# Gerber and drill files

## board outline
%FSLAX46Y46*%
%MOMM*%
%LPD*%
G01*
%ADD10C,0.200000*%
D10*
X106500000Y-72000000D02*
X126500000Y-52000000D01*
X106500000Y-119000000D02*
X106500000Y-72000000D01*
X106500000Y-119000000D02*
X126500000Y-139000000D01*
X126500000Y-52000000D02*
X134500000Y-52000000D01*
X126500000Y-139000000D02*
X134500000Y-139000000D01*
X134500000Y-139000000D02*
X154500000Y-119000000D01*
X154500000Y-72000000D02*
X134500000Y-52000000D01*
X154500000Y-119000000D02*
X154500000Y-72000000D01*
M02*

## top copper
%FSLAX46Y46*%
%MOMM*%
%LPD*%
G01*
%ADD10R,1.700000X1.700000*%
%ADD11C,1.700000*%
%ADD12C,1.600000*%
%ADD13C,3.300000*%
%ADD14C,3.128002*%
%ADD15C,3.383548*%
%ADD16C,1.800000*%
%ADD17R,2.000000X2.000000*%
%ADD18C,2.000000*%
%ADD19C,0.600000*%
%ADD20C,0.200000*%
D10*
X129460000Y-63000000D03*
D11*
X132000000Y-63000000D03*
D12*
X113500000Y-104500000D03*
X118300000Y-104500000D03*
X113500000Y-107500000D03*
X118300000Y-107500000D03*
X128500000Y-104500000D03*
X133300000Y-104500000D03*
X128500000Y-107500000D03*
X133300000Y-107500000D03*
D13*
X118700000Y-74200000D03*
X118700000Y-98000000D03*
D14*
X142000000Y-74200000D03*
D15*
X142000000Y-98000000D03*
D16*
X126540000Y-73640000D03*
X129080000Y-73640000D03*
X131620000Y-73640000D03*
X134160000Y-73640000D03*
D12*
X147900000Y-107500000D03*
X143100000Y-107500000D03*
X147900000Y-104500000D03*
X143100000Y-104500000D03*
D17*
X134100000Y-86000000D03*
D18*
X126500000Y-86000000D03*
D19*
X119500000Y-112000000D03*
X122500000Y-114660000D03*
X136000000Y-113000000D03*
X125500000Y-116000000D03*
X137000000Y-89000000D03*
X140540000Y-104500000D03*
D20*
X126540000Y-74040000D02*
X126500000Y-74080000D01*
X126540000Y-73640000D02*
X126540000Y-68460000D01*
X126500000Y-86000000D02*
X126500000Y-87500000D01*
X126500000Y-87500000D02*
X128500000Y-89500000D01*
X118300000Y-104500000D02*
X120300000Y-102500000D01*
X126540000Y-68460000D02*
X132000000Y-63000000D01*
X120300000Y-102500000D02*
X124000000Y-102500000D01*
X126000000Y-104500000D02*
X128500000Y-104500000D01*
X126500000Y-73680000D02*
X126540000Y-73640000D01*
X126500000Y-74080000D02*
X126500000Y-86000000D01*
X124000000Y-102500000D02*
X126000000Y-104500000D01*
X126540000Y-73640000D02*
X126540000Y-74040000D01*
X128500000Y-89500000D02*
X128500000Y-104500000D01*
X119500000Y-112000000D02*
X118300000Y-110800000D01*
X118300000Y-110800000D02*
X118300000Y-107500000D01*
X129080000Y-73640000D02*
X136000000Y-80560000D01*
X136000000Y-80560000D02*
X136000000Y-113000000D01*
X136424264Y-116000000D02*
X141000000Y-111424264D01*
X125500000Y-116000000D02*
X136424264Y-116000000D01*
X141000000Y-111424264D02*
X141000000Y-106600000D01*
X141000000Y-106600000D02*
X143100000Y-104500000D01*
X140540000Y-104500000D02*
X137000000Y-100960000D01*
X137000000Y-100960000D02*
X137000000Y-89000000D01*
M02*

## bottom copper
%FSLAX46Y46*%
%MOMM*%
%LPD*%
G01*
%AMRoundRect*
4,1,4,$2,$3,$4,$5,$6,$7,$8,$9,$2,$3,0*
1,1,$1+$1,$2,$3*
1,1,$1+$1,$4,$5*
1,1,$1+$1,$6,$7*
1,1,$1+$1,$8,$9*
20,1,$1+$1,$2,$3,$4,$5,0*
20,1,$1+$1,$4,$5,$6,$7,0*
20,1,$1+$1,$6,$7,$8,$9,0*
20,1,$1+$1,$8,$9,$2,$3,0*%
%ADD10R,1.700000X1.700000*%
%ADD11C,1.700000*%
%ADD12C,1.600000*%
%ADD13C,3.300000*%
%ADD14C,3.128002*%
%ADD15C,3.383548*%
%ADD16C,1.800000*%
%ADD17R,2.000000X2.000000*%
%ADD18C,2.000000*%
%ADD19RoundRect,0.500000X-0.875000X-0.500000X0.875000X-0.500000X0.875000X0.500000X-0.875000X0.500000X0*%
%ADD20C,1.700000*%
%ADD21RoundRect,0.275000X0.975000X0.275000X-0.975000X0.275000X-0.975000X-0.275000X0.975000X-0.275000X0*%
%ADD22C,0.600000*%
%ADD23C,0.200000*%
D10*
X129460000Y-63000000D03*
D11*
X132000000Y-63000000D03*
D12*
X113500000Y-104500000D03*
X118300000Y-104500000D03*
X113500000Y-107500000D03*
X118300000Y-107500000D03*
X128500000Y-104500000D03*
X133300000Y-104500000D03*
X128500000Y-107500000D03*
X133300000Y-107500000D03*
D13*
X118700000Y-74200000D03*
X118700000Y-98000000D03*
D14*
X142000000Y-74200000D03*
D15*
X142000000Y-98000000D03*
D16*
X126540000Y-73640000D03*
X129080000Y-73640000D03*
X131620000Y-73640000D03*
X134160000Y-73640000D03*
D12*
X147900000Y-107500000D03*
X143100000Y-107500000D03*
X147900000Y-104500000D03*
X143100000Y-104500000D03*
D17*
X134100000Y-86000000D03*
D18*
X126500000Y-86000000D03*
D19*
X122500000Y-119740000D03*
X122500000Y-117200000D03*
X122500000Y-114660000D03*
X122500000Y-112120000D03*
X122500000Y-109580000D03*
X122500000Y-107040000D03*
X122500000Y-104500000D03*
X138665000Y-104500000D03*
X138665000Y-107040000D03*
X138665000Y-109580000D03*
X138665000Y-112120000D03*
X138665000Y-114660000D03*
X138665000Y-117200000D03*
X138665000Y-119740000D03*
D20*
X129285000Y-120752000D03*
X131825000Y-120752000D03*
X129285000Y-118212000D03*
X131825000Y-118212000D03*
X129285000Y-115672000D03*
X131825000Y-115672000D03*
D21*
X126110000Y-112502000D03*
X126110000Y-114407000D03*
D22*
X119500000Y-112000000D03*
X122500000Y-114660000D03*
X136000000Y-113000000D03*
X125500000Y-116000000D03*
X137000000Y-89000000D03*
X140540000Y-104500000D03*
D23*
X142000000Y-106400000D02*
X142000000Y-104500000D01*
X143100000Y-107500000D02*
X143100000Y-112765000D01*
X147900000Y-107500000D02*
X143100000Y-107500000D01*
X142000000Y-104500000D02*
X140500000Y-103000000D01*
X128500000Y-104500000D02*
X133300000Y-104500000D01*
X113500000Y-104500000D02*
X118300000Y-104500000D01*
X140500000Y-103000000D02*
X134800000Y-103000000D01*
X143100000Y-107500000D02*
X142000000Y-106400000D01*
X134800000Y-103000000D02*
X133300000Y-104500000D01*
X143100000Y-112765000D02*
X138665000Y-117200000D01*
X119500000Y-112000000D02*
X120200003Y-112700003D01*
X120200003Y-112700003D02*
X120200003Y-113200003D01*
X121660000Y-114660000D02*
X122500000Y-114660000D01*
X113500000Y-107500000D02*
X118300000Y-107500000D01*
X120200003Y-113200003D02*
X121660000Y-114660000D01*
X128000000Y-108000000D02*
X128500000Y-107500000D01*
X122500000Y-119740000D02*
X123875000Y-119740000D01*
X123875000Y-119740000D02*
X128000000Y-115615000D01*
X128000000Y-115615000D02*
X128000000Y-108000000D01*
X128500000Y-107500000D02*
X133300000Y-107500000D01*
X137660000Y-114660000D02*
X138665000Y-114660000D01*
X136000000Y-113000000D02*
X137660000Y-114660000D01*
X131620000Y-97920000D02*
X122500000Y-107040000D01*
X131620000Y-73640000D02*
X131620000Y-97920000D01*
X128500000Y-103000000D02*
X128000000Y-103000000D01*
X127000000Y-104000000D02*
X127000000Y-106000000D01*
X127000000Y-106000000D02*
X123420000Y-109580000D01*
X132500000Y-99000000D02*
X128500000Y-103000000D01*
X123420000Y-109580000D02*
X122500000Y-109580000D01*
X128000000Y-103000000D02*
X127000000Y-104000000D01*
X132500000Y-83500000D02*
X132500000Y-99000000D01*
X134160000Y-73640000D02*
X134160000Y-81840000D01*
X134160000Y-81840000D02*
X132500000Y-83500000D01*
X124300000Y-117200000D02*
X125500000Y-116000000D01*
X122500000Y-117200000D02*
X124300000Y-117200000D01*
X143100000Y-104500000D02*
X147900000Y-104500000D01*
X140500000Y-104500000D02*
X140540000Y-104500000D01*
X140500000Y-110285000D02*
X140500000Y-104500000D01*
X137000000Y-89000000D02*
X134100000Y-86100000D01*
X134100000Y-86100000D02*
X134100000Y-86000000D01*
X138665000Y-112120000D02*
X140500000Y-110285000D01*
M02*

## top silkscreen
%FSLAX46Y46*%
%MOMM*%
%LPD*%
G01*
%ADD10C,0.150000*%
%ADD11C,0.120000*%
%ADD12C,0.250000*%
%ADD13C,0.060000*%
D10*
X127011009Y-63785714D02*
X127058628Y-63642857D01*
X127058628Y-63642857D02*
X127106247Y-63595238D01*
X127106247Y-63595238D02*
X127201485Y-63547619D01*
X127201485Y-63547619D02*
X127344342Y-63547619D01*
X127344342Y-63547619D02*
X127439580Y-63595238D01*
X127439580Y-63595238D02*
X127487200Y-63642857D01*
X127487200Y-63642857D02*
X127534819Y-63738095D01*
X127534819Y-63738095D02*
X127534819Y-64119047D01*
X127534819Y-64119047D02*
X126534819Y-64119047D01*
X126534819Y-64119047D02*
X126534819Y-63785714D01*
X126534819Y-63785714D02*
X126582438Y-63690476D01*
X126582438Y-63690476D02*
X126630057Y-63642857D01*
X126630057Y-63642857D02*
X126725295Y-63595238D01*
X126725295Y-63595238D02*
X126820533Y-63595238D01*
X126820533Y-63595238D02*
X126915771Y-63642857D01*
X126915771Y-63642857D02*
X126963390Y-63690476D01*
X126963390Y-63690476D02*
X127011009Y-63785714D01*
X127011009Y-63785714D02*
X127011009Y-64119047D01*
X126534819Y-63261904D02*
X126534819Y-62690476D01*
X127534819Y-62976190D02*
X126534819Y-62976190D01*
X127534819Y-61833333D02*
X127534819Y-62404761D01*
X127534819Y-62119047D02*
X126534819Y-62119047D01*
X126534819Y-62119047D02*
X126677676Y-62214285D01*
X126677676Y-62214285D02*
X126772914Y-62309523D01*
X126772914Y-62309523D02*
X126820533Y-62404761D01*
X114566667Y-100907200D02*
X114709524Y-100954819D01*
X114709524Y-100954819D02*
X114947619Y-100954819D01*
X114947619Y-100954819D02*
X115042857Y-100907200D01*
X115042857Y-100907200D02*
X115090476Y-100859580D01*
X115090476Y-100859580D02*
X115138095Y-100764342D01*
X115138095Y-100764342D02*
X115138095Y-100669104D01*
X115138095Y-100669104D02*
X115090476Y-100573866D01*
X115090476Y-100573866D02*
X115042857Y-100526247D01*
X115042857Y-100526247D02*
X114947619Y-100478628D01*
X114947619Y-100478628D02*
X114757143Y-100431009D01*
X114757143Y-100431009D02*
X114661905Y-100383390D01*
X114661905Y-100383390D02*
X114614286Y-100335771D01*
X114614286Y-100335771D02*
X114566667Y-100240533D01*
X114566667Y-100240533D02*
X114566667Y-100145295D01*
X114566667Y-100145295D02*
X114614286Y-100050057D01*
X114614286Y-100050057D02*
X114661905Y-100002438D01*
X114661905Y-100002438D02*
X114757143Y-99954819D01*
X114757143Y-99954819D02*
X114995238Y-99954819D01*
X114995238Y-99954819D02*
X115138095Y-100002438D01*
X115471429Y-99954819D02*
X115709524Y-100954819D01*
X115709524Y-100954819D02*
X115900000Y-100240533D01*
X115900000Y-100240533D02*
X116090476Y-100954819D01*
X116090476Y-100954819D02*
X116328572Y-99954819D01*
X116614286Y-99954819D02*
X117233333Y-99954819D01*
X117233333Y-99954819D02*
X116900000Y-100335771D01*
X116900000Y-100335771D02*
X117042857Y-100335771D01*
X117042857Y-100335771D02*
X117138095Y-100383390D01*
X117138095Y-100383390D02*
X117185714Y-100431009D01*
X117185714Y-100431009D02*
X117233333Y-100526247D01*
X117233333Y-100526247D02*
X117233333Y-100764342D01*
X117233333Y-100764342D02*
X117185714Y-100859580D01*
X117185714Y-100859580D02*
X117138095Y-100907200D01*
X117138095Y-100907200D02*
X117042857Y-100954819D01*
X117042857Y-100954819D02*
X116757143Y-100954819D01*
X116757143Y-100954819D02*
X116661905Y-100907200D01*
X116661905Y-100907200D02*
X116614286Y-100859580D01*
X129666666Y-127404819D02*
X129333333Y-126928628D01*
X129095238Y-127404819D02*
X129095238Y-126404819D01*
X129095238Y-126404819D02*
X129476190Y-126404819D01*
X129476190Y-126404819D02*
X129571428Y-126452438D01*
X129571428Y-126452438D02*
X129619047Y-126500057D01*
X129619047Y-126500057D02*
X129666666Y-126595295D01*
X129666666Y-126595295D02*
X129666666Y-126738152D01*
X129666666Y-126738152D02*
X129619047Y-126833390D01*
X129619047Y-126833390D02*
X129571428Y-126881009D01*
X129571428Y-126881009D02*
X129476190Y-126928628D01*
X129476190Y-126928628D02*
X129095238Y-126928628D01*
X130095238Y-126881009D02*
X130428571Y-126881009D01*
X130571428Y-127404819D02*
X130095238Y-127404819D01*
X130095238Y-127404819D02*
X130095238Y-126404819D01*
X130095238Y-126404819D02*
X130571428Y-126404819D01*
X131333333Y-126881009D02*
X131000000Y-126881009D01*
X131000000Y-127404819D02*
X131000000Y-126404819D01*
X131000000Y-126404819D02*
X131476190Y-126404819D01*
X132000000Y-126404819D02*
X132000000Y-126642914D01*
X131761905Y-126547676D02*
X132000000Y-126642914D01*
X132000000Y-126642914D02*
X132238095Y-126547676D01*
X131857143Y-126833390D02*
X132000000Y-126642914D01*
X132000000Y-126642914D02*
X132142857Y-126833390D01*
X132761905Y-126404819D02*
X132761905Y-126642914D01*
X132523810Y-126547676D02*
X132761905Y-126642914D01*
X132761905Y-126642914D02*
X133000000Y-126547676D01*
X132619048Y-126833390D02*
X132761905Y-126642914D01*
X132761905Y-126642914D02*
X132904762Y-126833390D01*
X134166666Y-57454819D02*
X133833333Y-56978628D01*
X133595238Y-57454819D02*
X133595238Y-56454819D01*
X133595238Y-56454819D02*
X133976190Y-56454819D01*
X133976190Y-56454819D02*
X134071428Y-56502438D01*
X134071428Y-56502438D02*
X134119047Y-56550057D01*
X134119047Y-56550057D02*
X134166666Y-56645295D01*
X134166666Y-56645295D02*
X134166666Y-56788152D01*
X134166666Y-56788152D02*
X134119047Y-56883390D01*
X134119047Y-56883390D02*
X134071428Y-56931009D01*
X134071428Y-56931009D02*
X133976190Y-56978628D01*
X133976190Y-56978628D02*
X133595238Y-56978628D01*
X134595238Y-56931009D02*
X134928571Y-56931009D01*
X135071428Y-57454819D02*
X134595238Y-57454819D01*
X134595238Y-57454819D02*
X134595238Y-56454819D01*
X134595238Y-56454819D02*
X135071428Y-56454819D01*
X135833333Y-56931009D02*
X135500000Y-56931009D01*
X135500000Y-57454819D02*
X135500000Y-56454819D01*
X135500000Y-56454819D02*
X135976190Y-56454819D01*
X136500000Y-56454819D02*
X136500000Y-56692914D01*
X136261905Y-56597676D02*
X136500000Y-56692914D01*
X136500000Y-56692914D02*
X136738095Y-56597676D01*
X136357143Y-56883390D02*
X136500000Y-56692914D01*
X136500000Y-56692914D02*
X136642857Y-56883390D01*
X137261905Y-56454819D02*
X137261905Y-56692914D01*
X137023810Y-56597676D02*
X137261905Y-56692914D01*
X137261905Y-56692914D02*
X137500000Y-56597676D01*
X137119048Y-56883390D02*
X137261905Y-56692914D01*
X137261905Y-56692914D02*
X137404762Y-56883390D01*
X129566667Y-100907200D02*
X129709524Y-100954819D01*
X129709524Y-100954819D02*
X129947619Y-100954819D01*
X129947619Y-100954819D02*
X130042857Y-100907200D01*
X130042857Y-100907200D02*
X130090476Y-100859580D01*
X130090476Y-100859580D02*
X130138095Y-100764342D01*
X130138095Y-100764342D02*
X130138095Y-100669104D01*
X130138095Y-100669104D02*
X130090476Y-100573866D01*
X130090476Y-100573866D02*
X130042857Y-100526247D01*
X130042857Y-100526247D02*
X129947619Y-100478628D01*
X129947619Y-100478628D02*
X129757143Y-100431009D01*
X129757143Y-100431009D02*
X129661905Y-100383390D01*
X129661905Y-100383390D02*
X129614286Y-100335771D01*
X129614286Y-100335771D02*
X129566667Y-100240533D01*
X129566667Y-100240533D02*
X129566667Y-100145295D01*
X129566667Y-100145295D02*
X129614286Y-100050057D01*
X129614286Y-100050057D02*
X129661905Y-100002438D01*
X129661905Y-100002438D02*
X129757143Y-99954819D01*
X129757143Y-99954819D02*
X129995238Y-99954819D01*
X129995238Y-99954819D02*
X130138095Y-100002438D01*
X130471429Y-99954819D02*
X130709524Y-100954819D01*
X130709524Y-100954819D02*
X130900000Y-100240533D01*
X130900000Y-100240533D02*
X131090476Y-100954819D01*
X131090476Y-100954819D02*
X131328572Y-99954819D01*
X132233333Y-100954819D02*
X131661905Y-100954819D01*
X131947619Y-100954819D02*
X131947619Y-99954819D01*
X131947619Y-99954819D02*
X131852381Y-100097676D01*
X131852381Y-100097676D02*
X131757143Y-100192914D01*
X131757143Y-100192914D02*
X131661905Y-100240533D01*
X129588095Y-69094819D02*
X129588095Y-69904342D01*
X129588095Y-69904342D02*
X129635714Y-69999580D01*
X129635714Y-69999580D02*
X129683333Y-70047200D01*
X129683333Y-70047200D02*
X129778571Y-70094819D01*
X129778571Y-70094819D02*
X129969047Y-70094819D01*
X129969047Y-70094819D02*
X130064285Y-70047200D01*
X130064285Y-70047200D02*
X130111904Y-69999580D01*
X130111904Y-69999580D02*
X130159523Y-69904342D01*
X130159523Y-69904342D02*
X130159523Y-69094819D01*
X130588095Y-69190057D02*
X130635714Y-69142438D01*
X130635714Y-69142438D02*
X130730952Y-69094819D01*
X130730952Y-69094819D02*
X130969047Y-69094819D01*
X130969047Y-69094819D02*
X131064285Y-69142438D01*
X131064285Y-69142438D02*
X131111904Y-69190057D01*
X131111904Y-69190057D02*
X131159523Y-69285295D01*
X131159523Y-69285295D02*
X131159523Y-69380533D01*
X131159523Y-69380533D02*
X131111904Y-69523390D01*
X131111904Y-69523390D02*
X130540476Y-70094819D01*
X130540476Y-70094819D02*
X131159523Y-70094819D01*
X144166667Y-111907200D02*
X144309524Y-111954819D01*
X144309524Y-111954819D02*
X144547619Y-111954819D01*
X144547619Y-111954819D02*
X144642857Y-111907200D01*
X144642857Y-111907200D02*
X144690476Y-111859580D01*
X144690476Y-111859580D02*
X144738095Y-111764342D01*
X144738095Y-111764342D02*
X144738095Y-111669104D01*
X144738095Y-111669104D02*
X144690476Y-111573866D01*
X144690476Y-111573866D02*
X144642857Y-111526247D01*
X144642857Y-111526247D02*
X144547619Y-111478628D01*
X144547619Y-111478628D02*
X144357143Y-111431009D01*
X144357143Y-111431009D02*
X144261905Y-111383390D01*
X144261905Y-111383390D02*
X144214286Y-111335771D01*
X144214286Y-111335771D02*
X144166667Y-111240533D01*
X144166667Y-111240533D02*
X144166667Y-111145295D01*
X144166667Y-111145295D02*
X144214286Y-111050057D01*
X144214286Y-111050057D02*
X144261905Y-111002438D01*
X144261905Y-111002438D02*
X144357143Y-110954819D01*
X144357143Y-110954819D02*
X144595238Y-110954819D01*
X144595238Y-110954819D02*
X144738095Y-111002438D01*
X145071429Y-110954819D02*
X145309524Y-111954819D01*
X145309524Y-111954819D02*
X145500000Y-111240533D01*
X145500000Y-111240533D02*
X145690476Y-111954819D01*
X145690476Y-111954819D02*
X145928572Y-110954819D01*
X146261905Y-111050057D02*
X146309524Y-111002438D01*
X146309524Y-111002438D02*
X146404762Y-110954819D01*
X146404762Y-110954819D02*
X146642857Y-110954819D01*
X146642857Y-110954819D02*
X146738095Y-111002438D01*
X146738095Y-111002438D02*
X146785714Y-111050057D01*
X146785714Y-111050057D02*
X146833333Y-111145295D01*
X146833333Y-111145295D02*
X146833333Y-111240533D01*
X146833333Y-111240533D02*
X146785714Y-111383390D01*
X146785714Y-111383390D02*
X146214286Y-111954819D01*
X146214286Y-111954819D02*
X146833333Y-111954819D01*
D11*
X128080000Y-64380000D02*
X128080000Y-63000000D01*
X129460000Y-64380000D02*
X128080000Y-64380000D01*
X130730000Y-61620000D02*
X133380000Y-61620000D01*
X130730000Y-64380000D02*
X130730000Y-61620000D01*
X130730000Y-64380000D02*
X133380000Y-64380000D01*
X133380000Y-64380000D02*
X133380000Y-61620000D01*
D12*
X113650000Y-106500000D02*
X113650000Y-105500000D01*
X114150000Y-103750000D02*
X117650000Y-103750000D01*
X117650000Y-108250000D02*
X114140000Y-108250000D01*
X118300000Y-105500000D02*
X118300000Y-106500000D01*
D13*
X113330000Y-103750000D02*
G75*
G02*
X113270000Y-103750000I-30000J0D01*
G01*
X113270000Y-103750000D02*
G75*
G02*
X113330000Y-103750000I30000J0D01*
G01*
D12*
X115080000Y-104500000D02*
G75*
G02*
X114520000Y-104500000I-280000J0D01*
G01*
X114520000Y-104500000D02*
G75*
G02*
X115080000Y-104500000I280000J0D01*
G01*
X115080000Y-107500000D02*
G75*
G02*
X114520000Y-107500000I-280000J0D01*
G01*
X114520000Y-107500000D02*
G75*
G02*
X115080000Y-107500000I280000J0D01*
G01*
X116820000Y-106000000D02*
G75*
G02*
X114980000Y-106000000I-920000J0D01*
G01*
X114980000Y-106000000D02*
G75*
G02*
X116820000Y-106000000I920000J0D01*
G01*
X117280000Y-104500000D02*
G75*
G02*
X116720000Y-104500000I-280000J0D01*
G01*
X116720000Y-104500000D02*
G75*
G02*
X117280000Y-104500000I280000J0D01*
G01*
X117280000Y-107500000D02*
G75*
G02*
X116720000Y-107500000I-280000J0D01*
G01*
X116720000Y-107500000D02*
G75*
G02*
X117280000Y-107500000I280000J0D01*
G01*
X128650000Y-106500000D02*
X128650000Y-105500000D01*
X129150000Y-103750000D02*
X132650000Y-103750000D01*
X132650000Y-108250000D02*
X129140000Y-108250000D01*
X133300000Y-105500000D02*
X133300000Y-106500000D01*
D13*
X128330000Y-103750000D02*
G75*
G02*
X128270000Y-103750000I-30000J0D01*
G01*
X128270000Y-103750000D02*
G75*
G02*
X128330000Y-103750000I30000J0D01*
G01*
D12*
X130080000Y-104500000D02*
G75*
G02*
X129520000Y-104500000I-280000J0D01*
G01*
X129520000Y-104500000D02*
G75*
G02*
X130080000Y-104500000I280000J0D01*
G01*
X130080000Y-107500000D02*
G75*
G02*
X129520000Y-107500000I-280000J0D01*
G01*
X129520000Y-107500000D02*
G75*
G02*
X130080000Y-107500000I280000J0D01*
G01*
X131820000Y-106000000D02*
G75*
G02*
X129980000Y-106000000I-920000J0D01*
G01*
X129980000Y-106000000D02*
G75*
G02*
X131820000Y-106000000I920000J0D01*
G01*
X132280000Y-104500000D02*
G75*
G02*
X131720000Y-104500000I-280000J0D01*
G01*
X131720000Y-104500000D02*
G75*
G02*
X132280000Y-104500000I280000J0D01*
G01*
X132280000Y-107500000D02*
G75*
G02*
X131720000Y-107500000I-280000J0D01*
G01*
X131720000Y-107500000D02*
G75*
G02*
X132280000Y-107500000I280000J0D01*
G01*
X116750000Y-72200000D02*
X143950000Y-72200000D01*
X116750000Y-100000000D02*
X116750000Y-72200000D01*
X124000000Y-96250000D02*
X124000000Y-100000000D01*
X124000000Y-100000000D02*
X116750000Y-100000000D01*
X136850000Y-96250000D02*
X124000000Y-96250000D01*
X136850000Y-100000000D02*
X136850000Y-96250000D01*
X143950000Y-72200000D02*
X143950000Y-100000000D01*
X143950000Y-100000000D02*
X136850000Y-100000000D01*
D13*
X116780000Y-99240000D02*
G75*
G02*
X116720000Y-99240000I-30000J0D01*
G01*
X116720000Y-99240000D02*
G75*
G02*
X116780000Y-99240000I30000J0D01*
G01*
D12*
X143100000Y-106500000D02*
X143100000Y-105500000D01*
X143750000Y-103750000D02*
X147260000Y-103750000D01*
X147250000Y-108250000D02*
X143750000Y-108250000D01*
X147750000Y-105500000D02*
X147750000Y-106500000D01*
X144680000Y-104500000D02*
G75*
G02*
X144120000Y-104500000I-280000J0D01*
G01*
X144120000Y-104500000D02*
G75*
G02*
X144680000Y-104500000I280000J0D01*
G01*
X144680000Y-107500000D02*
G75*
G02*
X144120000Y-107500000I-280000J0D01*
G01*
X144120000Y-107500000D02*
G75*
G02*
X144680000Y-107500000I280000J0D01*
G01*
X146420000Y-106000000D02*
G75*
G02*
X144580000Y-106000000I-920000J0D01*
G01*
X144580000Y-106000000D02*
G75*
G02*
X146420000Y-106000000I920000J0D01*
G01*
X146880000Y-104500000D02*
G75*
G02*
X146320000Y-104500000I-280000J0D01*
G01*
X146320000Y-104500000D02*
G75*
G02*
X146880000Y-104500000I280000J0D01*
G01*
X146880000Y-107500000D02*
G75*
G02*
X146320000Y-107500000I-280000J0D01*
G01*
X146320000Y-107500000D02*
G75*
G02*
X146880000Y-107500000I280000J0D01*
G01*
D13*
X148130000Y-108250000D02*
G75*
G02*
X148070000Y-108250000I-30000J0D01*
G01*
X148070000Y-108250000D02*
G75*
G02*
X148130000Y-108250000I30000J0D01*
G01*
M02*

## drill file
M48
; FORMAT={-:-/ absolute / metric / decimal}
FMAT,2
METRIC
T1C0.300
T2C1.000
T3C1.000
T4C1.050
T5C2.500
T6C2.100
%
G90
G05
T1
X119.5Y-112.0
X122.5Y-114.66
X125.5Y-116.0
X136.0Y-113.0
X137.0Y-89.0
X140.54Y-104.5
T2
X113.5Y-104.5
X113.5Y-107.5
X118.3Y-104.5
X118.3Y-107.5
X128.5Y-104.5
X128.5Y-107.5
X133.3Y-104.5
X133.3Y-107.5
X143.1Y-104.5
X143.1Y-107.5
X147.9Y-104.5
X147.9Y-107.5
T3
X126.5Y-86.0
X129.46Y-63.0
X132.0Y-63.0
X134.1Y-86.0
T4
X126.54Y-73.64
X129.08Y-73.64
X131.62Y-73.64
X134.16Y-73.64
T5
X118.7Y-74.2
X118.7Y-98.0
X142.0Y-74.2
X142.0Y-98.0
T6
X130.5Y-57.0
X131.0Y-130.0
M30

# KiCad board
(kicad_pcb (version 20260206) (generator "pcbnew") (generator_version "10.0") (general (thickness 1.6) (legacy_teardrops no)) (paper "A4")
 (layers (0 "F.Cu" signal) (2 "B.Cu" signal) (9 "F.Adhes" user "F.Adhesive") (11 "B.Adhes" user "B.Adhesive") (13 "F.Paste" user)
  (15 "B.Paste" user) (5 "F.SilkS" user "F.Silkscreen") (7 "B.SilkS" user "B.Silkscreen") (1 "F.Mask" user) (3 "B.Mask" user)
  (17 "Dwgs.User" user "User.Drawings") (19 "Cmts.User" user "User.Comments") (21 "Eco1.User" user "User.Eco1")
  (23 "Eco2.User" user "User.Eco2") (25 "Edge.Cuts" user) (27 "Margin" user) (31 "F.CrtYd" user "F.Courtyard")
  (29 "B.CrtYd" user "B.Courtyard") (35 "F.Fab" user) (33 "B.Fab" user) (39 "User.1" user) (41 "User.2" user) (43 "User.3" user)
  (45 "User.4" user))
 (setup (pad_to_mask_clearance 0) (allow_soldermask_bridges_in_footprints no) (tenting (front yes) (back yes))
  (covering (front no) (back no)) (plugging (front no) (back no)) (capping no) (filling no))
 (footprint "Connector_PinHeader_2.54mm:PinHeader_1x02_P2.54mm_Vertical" (layer "F.Cu") (at 129.46 63 90)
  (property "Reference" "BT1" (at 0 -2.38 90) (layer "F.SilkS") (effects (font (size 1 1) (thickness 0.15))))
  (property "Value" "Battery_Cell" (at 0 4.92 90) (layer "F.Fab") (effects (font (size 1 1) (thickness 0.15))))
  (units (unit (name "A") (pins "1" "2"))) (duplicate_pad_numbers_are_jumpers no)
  (fp_line (start -1.38 -1.38) (end 0 -1.38) (stroke (width 0.12) (type solid)) (layer "F.SilkS"))
  (fp_line (start -1.38 0) (end -1.38 -1.38) (stroke (width 0.12) (type solid)) (layer "F.SilkS"))
  (fp_line (start 1.38 1.27) (end 1.38 3.92) (stroke (width 0.12) (type solid)) (layer "F.SilkS"))
  (fp_line (start -1.38 1.27) (end 1.38 1.27) (stroke (width 0.12) (type solid)) (layer "F.SilkS"))
  (fp_line (start -1.38 1.27) (end -1.38 3.92) (stroke (width 0.12) (type solid)) (layer "F.SilkS"))
  (fp_line (start -1.38 3.92) (end 1.38 3.92) (stroke (width 0.12) (type solid)) (layer "F.SilkS"))
  (pad "1" thru_hole rect (at 0 0 90) (size 1.7 1.7) (drill 1) (layers "*.Cu" "*.Mask") (remove_unused_layers no) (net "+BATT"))
  (pad "2" thru_hole circle (at 0 2.54 90) (size 1.7 1.7) (drill 1) (layers "*.Cu" "*.Mask") (remove_unused_layers no) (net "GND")))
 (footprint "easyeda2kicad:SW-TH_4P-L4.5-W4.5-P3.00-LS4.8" (layer "F.Cu") (at 115.9 106)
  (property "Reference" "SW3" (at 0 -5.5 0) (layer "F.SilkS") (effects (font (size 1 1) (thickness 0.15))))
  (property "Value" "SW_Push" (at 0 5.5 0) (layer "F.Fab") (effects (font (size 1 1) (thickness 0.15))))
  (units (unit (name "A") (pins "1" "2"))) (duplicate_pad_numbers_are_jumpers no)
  (fp_line (start -2.25 0.5) (end -2.25 -0.5) (stroke (width 0.25) (type solid)) (layer "F.SilkS"))
  (fp_line (start -1.75 -2.25) (end 1.75 -2.25) (stroke (width 0.25) (type solid)) (layer "F.SilkS"))
  (fp_line (start 1.75 2.25) (end -1.76 2.25) (stroke (width 0.25) (type solid)) (layer "F.SilkS"))
  (fp_line (start 2.4 -0.5) (end 2.4 0.5) (stroke (width 0.25) (type solid)) (layer "F.SilkS"))
  (fp_circle (center -2.6 -2.25) (end -2.57 -2.25) (stroke (width 0.06) (type solid)) (fill no) (layer "F.SilkS"))
  (fp_circle (center -1.1 -1.5) (end -0.82 -1.5) (stroke (width 0.25) (type solid)) (fill no) (layer "F.SilkS"))
  (fp_circle (center -1.1 1.5) (end -0.82 1.5) (stroke (width 0.25) (type solid)) (fill no) (layer "F.SilkS"))
  (fp_circle (center 0 0) (end 0.92 0) (stroke (width 0.25) (type solid)) (fill no) (layer "F.SilkS"))
  (fp_circle (center 1.1 -1.5) (end 1.38 -1.5) (stroke (width 0.25) (type solid)) (fill no) (layer "F.SilkS"))
  (fp_circle (center 1.1 1.5) (end 1.38 1.5) (stroke (width 0.25) (type solid)) (fill no) (layer "F.SilkS"))
  (pad "1" thru_hole circle (at -2.4 -1.5) (size 1.6 1.6) (drill 0.999998) (layers "*.Cu" "*.Mask") (remove_unused_layers no) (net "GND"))
  (pad "1" thru_hole circle (at 2.4 -1.5) (size 1.6 1.6) (drill 0.999998) (layers "*.Cu" "*.Mask") (remove_unused_layers no) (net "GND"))
  (pad "2" thru_hole circle (at -2.4 1.5) (size 1.6 1.6) (drill 0.999998) (layers "*.Cu" "*.Mask") (remove_unused_layers no)
   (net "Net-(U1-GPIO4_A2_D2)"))
  (pad "2" thru_hole circle (at 2.4 1.5) (size 1.6 1.6) (drill 0.999998) (layers "*.Cu" "*.Mask") (remove_unused_layers no)
   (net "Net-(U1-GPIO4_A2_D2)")))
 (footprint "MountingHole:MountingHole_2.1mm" (layer "F.Cu") (at 131 130)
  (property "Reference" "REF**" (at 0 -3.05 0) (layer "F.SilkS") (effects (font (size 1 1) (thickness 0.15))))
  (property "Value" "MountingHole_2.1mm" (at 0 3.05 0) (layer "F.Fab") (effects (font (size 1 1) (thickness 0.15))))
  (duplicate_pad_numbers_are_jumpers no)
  (pad "" np_thru_hole circle (at 0 0) (size 2.1 2.1) (drill 2.1) (layers "*.Cu" "*.Mask")))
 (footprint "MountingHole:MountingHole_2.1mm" (layer "F.Cu") (at 130.5 57)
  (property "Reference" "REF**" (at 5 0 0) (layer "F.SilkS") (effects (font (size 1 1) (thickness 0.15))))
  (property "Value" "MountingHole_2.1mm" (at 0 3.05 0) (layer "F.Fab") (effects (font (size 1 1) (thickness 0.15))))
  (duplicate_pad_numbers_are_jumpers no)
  (pad "" np_thru_hole circle (at 0 0) (size 2.1 2.1) (drill 2.1) (layers "*.Cu" "*.Mask")))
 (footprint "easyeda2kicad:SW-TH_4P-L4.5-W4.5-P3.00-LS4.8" (layer "F.Cu") (at 130.9 106)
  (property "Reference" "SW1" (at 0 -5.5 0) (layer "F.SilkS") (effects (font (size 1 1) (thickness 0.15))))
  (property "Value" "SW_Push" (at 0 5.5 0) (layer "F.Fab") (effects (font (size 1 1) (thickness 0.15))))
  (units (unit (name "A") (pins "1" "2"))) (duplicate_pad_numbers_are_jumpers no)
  (fp_line (start -2.25 0.5) (end -2.25 -0.5) (stroke (width 0.25) (type solid)) (layer "F.SilkS"))
  (fp_line (start -1.75 -2.25) (end 1.75 -2.25) (stroke (width 0.25) (type solid)) (layer "F.SilkS"))
  (fp_line (start 1.75 2.25) (end -1.76 2.25) (stroke (width 0.25) (type solid)) (layer "F.SilkS"))
  (fp_line (start 2.4 -0.5) (end 2.4 0.5) (stroke (width 0.25) (type solid)) (layer "F.SilkS"))
  (fp_circle (center -2.6 -2.25) (end -2.57 -2.25) (stroke (width 0.06) (type solid)) (fill no) (layer "F.SilkS"))
  (fp_circle (center -1.1 -1.5) (end -0.82 -1.5) (stroke (width 0.25) (type solid)) (fill no) (layer "F.SilkS"))
  (fp_circle (center -1.1 1.5) (end -0.82 1.5) (stroke (width 0.25) (type solid)) (fill no) (layer "F.SilkS"))
  (fp_circle (center 0 0) (end 0.92 0) (stroke (width 0.25) (type solid)) (fill no) (layer "F.SilkS"))
  (fp_circle (center 1.1 -1.5) (end 1.38 -1.5) (stroke (width 0.25) (type solid)) (fill no) (layer "F.SilkS"))
  (fp_circle (center 1.1 1.5) (end 1.38 1.5) (stroke (width 0.25) (type solid)) (fill no) (layer "F.SilkS"))
  (pad "1" thru_hole circle (at -2.4 -1.5) (size 1.6 1.6) (drill 0.999998) (layers "*.Cu" "*.Mask") (remove_unused_layers no) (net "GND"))
  (pad "1" thru_hole circle (at 2.4 -1.5) (size 1.6 1.6) (drill 0.999998) (layers "*.Cu" "*.Mask") (remove_unused_layers no) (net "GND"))
  (pad "2" thru_hole circle (at -2.4 1.5) (size 1.6 1.6) (drill 0.999998) (layers "*.Cu" "*.Mask") (remove_unused_layers no)
   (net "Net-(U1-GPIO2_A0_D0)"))
  (pad "2" thru_hole circle (at 2.4 1.5) (size 1.6 1.6) (drill 0.999998) (layers "*.Cu" "*.Mask") (remove_unused_layers no)
   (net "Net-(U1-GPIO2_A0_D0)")))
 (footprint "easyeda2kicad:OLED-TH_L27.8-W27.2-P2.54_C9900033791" (layer "F.Cu") (at 130.35 73.64)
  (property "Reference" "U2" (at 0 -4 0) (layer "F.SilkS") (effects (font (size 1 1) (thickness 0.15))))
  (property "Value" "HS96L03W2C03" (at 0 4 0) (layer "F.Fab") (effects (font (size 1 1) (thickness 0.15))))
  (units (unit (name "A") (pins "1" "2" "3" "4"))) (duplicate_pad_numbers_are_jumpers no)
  (fp_line (start -13.6 -1.44) (end 13.6 -1.44) (stroke (width 0.25) (type solid)) (layer "F.SilkS"))
  (fp_line (start -13.6 26.36) (end -13.6 -1.44) (stroke (width 0.25) (type solid)) (layer "F.SilkS"))
  (fp_line (start -6.35 22.61) (end -6.35 26.36) (stroke (width 0.25) (type solid)) (layer "F.SilkS"))
  (fp_line (start -6.35 26.36) (end -13.6 26.36) (stroke (width 0.25) (type solid)) (layer "F.SilkS"))
  (fp_line (start 6.5 22.61) (end -6.35 22.61) (stroke (width 0.25) (type solid)) (layer "F.SilkS"))
  (fp_line (start 6.5 26.36) (end 6.5 22.61) (stroke (width 0.25) (type solid)) (layer "F.SilkS"))
  (fp_line (start 13.6 -1.44) (end 13.6 26.36) (stroke (width 0.25) (type solid)) (layer "F.SilkS"))
  (fp_line (start 13.6 26.36) (end 6.5 26.36) (stroke (width 0.25) (type solid)) (layer "F.SilkS"))
  (fp_circle (center -13.6 25.6) (end -13.57 25.6) (stroke (width 0.06) (type solid)) (fill no) (layer "F.SilkS"))
  (pad "" thru_hole circle (at -11.65 0.56) (size 3.3 3.3) (drill 2.5) (layers "*.Cu" "*.Mask") (remove_unused_layers no))
  (pad "" thru_hole circle (at -11.65 24.36) (size 3.3 3.3) (drill 2.5) (layers "*.Cu" "*.Mask") (remove_unused_layers no))
  (pad "" thru_hole circle (at 11.65 0.56) (size 3.128002 3.128002) (drill 2.5) (layers "*.Cu" "*.Mask") (remove_unused_layers no))
  (pad "" thru_hole circle (at 11.65 24.36) (size 3.383548 3.383548) (drill 2.5) (layers "*.Cu" "*.Mask") (remove_unused_layers no))
  (pad "1" thru_hole circle (at -3.81 0) (size 1.8 1.8) (drill 1.049986) (layers "*.Cu" "*.Mask") (remove_unused_layers no) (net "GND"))
  (pad "2" thru_hole circle (at -1.27 0) (size 1.8 1.8) (drill 1.049986) (layers "*.Cu" "*.Mask") (remove_unused_layers no) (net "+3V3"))
  (pad "3" thru_hole circle (at 1.27 0) (size 1.8 1.8) (drill 1.049986) (layers "*.Cu" "*.Mask") (remove_unused_layers no)
   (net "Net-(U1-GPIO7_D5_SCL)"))
  (pad "4" thru_hole circle (at 3.81 0) (size 1.8 1.8) (drill 1.049986) (layers "*.Cu" "*.Mask") (remove_unused_layers no)
   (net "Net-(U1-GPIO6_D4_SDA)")))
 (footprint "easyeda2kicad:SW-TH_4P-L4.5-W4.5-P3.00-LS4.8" (layer "F.Cu") (at 145.5 106 180)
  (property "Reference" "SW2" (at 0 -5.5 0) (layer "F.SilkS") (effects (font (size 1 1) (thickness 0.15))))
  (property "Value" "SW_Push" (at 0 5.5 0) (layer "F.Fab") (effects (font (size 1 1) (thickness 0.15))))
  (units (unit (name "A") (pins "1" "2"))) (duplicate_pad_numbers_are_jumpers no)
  (fp_line (start 2.4 -0.5) (end 2.4 0.5) (stroke (width 0.25) (type solid)) (layer "F.SilkS"))
  (fp_line (start 1.75 2.25) (end -1.76 2.25) (stroke (width 0.25) (type solid)) (layer "F.SilkS"))
  (fp_line (start -1.75 -2.25) (end 1.75 -2.25) (stroke (width 0.25) (type solid)) (layer "F.SilkS"))
  (fp_line (start -2.25 0.5) (end -2.25 -0.5) (stroke (width 0.25) (type solid)) (layer "F.SilkS"))
  (fp_circle (center 1.1 1.5) (end 1.38 1.5) (stroke (width 0.25) (type solid)) (fill no) (layer "F.SilkS"))
  (fp_circle (center 1.1 -1.5) (end 1.38 -1.5) (stroke (width 0.25) (type solid)) (fill no) (layer "F.SilkS"))
  (fp_circle (center 0 0) (end 0.92 0) (stroke (width 0.25) (type solid)) (fill no) (layer "F.SilkS"))
  (fp_circle (center -1.1 1.5) (end -0.82 1.5) (stroke (width 0.25) (type solid)) (fill no) (layer "F.SilkS"))
  (fp_circle (center -1.1 -1.5) (end -0.82 -1.5) (stroke (width 0.25) (type solid)) (fill no) (layer "F.SilkS"))
  (fp_circle (center -2.6 -2.25) (end -2.57 -2.25) (stroke (width 0.06) (type solid)) (fill no) (layer "F.SilkS"))
  (pad "1" thru_hole circle (at -2.4 -1.5 180) (size 1.6 1.6) (drill 0.999998) (layers "*.Cu" "*.Mask") (remove_unused_layers no)
   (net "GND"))
  (pad "1" thru_hole circle (at 2.4 -1.5 180) (size 1.6 1.6) (drill 0.999998) (layers "*.Cu" "*.Mask") (remove_unused_layers no) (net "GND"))
  (pad "2" thru_hole circle (at -2.4 1.5 180) (size 1.6 1.6) (drill 0.999998) (layers "*.Cu" "*.Mask") (remove_unused_layers no)
   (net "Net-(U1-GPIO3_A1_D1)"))
  (pad "2" thru_hole circle (at 2.4 1.5 180) (size 1.6 1.6) (drill 0.999998) (layers "*.Cu" "*.Mask") (remove_unused_layers no)
   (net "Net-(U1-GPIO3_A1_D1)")))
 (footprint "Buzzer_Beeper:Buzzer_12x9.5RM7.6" (layer "B.Cu") (at 134.1 86 180)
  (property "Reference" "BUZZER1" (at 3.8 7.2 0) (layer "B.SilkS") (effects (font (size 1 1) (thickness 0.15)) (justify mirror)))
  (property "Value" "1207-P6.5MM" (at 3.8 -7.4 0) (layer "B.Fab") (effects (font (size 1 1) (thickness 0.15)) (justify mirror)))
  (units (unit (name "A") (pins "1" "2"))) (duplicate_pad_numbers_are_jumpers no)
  (pad "1" thru_hole rect (at 0 0 180) (size 2 2) (drill 1) (layers "*.Cu" "*.Mask") (remove_unused_layers no) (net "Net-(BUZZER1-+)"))
  (pad "2" thru_hole circle (at 7.6 0 180) (size 2 2) (drill 1) (layers "*.Cu" "*.Mask") (remove_unused_layers no) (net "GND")))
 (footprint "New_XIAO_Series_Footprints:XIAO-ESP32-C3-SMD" (layer "B.Cu") (at 121.665 101.62)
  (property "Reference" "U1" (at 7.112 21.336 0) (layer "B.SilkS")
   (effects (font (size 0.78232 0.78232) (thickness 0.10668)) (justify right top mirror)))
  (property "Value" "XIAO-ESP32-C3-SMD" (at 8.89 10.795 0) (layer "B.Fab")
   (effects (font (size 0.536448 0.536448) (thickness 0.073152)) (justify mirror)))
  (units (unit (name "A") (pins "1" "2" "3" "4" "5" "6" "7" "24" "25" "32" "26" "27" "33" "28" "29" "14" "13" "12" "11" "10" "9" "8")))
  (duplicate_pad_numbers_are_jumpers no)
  (pad "1" smd roundrect (at 0.835 18.12) (size 2.75 2) (layers "B.Cu" "B.Mask" "B.Paste") (roundrect_rratio 0.25)
   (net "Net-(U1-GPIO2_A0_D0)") (solder_mask_margin 0.0508) (thermal_bridge_angle 45))
  (pad "2" smd roundrect (at 0.835 15.58) (size 2.75 2) (layers "B.Cu" "B.Mask" "B.Paste") (roundrect_rratio 0.25)
   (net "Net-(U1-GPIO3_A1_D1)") (solder_mask_margin 0.0508) (thermal_bridge_angle 45))
  (pad "3" smd roundrect (at 0.835 13.04) (size 2.75 2) (layers "B.Cu" "B.Mask" "B.Paste") (roundrect_rratio 0.25)
   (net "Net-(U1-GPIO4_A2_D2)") (solder_mask_margin 0.0508) (thermal_bridge_angle 45))
  (pad "4" smd roundrect (at 0.835 10.5) (size 2.75 2) (layers "B.Cu" "B.Mask" "B.Paste") (roundrect_rratio 0.25)
   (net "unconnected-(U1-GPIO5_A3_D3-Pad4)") (solder_mask_margin 0.0508) (thermal_bridge_angle 45))
  (pad "5" smd roundrect (at 0.835 7.96) (size 2.75 2) (layers "B.Cu" "B.Mask" "B.Paste") (roundrect_rratio 0.25)
   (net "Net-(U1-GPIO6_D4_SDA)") (solder_mask_margin 0.0508) (thermal_bridge_angle 45))
  (pad "6" smd roundrect (at 0.835 5.42) (size 2.75 2) (layers "B.Cu" "B.Mask" "B.Paste") (roundrect_rratio 0.25)
   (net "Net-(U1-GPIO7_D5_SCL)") (solder_mask_margin 0.0508) (thermal_bridge_angle 45))
  (pad "7" smd roundrect (at 0.835 2.88) (size 2.75 2) (layers "B.Cu" "B.Mask" "B.Paste") (roundrect_rratio 0.25)
   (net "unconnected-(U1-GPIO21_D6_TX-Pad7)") (solder_mask_margin 0.0508) (thermal_bridge_angle 45))
  (pad "8" smd roundrect (at 17 2.88) (size 2.75 2) (layers "B.Cu" "B.Mask" "B.Paste") (roundrect_rratio 0.25)
   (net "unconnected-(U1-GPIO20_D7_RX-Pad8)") (solder_mask_margin 0.0508) (thermal_bridge_angle 45))
  (pad "9" smd roundrect (at 17 5.42) (size 2.75 2) (layers "B.Cu" "B.Mask" "B.Paste") (roundrect_rratio 0.25)
   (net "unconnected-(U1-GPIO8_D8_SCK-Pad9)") (solder_mask_margin 0.0508) (thermal_bridge_angle 45))
  (pad "10" smd roundrect (at 17 7.96) (size 2.75 2) (layers "B.Cu" "B.Mask" "B.Paste") (roundrect_rratio 0.25)
   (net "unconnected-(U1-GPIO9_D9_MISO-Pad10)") (solder_mask_margin 0.0508) (thermal_bridge_angle 45))
  (pad "11" smd roundrect (at 17 10.5) (size 2.75 2) (layers "B.Cu" "B.Mask" "B.Paste") (roundrect_rratio 0.25) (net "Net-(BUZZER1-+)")
   (solder_mask_margin 0.0508) (thermal_bridge_angle 45))
  (pad "12" smd roundrect (at 17 13.04) (size 2.75 2) (layers "B.Cu" "B.Mask" "B.Paste") (roundrect_rratio 0.25) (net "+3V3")
   (solder_mask_margin 0.0508) (thermal_bridge_angle 45))
  (pad "13" smd roundrect (at 17 15.58) (size 2.75 2) (layers "B.Cu" "B.Mask" "B.Paste") (roundrect_rratio 0.25) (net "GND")
   (solder_mask_margin 0.0508) (thermal_bridge_angle 45))
  (pad "14" smd roundrect (at 17 18.12) (size 2.75 2) (layers "B.Cu" "B.Mask" "B.Paste") (roundrect_rratio 0.25) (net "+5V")
   (solder_mask_margin 0.0508) (thermal_bridge_angle 45))
  (pad "15" smd circle (at 7.62 19.132) (size 1.7 1.7) (layers "B.Cu" "B.Mask" "B.Paste"))
  (pad "16" smd circle (at 10.16 19.132) (size 1.7 1.7) (layers "B.Cu" "B.Mask" "B.Paste"))
  (pad "17" smd circle (at 7.62 16.592) (size 1.7 1.7) (layers "B.Cu" "B.Mask" "B.Paste"))
  (pad "18" smd circle (at 10.16 16.592) (size 1.7 1.7) (layers "B.Cu" "B.Mask" "B.Paste"))
  (pad "19" smd circle (at 7.62 14.052) (size 1.7 1.7) (layers "B.Cu" "B.Mask" "B.Paste"))
  (pad "20" smd circle (at 10.16 14.052) (size 1.7 1.7) (layers "B.Cu" "B.Mask" "B.Paste"))
  (pad "21" smd roundrect (at 4.445 10.882 180) (size 2.5 1.1) (layers "B.Cu" "B.Mask" "B.Paste") (roundrect_rratio 0.25)
   (thermal_bridge_angle 45))
  (pad "22" smd roundrect (at 4.445 12.787 180) (size 2.5 1.1) (layers "B.Cu" "B.Mask" "B.Paste") (roundrect_rratio 0.25)
   (thermal_bridge_angle 45)))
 (gr_line (start 106.5 72) (end 126.5 52) (stroke (width 0.2) (type default)) (layer "Edge.Cuts"))
 (gr_line (start 106.5 119) (end 106.5 72) (stroke (width 0.2) (type default)) (layer "Edge.Cuts"))
 (gr_line (start 106.5 119) (end 126.5 139) (stroke (width 0.2) (type default)) (layer "Edge.Cuts"))
 (gr_line (start 126.5 52) (end 134.5 52) (stroke (width 0.2) (type default)) (layer "Edge.Cuts"))
 (gr_line (start 126.5 139) (end 134.5 139) (stroke (width 0.2) (type default)) (layer "Edge.Cuts"))
 (gr_line (start 134.5 139) (end 154.5 119) (stroke (width 0.2) (type default)) (layer "Edge.Cuts"))
 (gr_line (start 154.5 72) (end 134.5 52) (stroke (width 0.2) (type default)) (layer "Edge.Cuts"))
 (gr_line (start 154.5 119) (end 154.5 72) (stroke (width 0.2) (type default)) (layer "Edge.Cuts"))
 (segment (start 126.54 74.04) (end 126.5 74.08) (width 0.2) (layer "F.Cu") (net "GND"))
 (segment (start 126.54 73.64) (end 126.54 68.46) (width 0.2) (layer "F.Cu") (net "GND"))
 (segment (start 126.5 86) (end 126.5 87.5) (width 0.2) (layer "F.Cu") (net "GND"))
 (segment (start 126.5 87.5) (end 128.5 89.5) (width 0.2) (layer "F.Cu") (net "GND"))
 (segment (start 118.3 104.5) (end 120.3 102.5) (width 0.2) (layer "F.Cu") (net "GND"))
 (segment (start 126.54 68.46) (end 132 63) (width 0.2) (layer "F.Cu") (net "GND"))
 (segment (start 120.3 102.5) (end 124 102.5) (width 0.2) (layer "F.Cu") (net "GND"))
 (segment (start 126 104.5) (end 128.5 104.5) (width 0.2) (layer "F.Cu") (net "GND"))
 (segment (start 126.5 73.68) (end 126.54 73.64) (width 0.2) (layer "F.Cu") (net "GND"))
 (segment (start 126.5 74.08) (end 126.5 86) (width 0.2) (layer "F.Cu") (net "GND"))
 (segment (start 124 102.5) (end 126 104.5) (width 0.2) (layer "F.Cu") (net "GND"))
 (segment (start 126.54 73.64) (end 126.54 74.04) (width 0.2) (layer "F.Cu") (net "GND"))
 (segment (start 128.5 89.5) (end 128.5 104.5) (width 0.2) (layer "F.Cu") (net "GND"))
 (segment (start 142 106.4) (end 142 104.5) (width 0.2) (layer "B.Cu") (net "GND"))
 (segment (start 143.1 107.5) (end 143.1 112.765) (width 0.2) (layer "B.Cu") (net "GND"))
 (segment (start 147.9 107.5) (end 143.1 107.5) (width 0.2) (layer "B.Cu") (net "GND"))
 (segment (start 142 104.5) (end 140.5 103) (width 0.2) (layer "B.Cu") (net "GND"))
 (segment (start 128.5 104.5) (end 133.3 104.5) (width 0.2) (layer "B.Cu") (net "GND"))
 (segment (start 113.5 104.5) (end 118.3 104.5) (width 0.2) (layer "B.Cu") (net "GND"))
 (segment (start 140.5 103) (end 134.8 103) (width 0.2) (layer "B.Cu") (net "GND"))
 (segment (start 143.1 107.5) (end 142 106.4) (width 0.2) (layer "B.Cu") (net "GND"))
 (segment (start 134.8 103) (end 133.3 104.5) (width 0.2) (layer "B.Cu") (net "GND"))
 (segment (start 143.1 112.765) (end 138.665 117.2) (width 0.2) (layer "B.Cu") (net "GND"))
 (segment (start 119.5 112) (end 118.3 110.8) (width 0.2) (layer "F.Cu") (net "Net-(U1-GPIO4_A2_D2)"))
 (segment (start 118.3 110.8) (end 118.3 107.5) (width 0.2) (layer "F.Cu") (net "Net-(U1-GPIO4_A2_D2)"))
 (via (at 119.5 112) (size 0.6) (drill 0.3) (layers "F.Cu" "B.Cu") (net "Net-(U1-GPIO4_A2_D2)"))
 (via (at 122.5 114.66) (size 0.6) (drill 0.3) (layers "F.Cu" "B.Cu") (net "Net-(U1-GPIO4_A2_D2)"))
 (segment (start 119.5 112) (end 120.200003 112.700003) (width 0.2) (layer "B.Cu") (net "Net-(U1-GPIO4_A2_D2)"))
 (segment (start 120.200003 112.700003) (end 120.200003 113.200003) (width 0.2) (layer "B.Cu") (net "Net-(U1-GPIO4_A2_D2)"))
 (segment (start 121.66 114.66) (end 122.5 114.66) (width 0.2) (layer "B.Cu") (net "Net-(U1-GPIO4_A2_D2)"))
 (segment (start 113.5 107.5) (end 118.3 107.5) (width 0.2) (layer "B.Cu") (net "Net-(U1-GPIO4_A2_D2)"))
 (segment (start 120.200003 113.200003) (end 121.66 114.66) (width 0.2) (layer "B.Cu") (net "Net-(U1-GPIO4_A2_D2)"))
 (segment (start 128 108) (end 128.5 107.5) (width 0.2) (layer "B.Cu") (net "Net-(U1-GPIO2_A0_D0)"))
 (segment (start 122.5 119.74) (end 123.875 119.74) (width 0.2) (layer "B.Cu") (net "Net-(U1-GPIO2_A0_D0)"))
 (segment (start 123.875 119.74) (end 128 115.615) (width 0.2) (layer "B.Cu") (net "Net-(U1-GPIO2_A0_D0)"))
 (segment (start 128 115.615) (end 128 108) (width 0.2) (layer "B.Cu") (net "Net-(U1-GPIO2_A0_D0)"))
 (segment (start 128.5 107.5) (end 133.3 107.5) (width 0.2) (layer "B.Cu") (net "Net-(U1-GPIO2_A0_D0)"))
 (segment (start 129.08 73.64) (end 136 80.56) (width 0.2) (layer "F.Cu") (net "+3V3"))
 (segment (start 136 80.56) (end 136 113) (width 0.2) (layer "F.Cu") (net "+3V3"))
 (via (at 136 113) (size 0.6) (drill 0.3) (layers "F.Cu" "B.Cu") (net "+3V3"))
 (segment (start 137.66 114.66) (end 138.665 114.66) (width 0.2) (layer "B.Cu") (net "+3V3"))
 (segment (start 136 113) (end 137.66 114.66) (width 0.2) (layer "B.Cu") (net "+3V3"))
 (segment (start 131.62 97.92) (end 122.5 107.04) (width 0.2) (layer "B.Cu") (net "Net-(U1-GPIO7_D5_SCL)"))
 (segment (start 131.62 73.64) (end 131.62 97.92) (width 0.2) (layer "B.Cu") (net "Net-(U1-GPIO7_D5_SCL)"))
 (segment (start 128.5 103) (end 128 103) (width 0.2) (layer "B.Cu") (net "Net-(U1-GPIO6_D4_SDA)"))
 (segment (start 127 104) (end 127 106) (width 0.2) (layer "B.Cu") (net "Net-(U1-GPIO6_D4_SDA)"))
 (segment (start 127 106) (end 123.42 109.58) (width 0.2) (layer "B.Cu") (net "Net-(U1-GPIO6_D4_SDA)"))
 (segment (start 132.5 99) (end 128.5 103) (width 0.2) (layer "B.Cu") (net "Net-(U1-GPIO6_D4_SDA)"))
 (segment (start 123.42 109.58) (end 122.5 109.58) (width 0.2) (layer "B.Cu") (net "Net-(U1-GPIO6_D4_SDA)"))
 (segment (start 128 103) (end 127 104) (width 0.2) (layer "B.Cu") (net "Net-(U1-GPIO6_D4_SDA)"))
 (segment (start 132.5 83.5) (end 132.5 99) (width 0.2) (layer "B.Cu") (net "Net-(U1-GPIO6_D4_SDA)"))
 (segment (start 134.16 73.64) (end 134.16 81.84) (width 0.2) (layer "B.Cu") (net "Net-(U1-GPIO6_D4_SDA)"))
 (segment (start 134.16 81.84) (end 132.5 83.5) (width 0.2) (layer "B.Cu") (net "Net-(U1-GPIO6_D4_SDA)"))
 (segment (start 136.424264 116) (end 141 111.424264) (width 0.2) (layer "F.Cu") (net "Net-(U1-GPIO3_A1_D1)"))
 (segment (start 125.5 116) (end 136.424264 116) (width 0.2) (layer "F.Cu") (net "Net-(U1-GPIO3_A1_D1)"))
 (segment (start 141 111.424264) (end 141 106.6) (width 0.2) (layer "F.Cu") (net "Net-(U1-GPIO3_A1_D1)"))
 (segment (start 141 106.6) (end 143.1 104.5) (width 0.2) (layer "F.Cu") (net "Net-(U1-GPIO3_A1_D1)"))
 (via (at 125.5 116) (size 0.6) (drill 0.3) (layers "F.Cu" "B.Cu") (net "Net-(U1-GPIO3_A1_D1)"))
 (segment (start 124.3 117.2) (end 125.5 116) (width 0.2) (layer "B.Cu") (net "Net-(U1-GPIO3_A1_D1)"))
 (segment (start 122.5 117.2) (end 124.3 117.2) (width 0.2) (layer "B.Cu") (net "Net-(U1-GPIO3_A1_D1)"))
 (segment (start 143.1 104.5) (end 147.9 104.5) (width 0.2) (layer "B.Cu") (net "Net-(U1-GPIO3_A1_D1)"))
 (segment (start 140.54 104.5) (end 137 100.96) (width 0.2) (layer "F.Cu") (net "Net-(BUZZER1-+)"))
 (segment (start 137 100.96) (end 137 89) (width 0.2) (layer "F.Cu") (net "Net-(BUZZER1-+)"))
 (via (at 137 89) (size 0.6) (drill 0.3) (layers "F.Cu" "B.Cu") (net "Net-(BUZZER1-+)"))
 (via (at 140.54 104.5) (size 0.6) (drill 0.3) (layers "F.Cu" "B.Cu") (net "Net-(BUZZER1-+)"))
 (segment (start 140.5 104.5) (end 140.54 104.5) (width 0.2) (layer "B.Cu") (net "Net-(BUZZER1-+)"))
 (segment (start 140.5 110.285) (end 140.5 104.5) (width 0.2) (layer "B.Cu") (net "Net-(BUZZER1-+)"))
 (segment (start 137 89) (end 134.1 86.1) (width 0.2) (layer "B.Cu") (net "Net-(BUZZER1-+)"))
 (segment (start 134.1 86.1) (end 134.1 86) (width 0.2) (layer "B.Cu") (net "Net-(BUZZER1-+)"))
 (segment (start 138.665 112.12) (end 140.5 110.285) (width 0.2) (layer "B.Cu") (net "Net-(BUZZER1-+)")))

